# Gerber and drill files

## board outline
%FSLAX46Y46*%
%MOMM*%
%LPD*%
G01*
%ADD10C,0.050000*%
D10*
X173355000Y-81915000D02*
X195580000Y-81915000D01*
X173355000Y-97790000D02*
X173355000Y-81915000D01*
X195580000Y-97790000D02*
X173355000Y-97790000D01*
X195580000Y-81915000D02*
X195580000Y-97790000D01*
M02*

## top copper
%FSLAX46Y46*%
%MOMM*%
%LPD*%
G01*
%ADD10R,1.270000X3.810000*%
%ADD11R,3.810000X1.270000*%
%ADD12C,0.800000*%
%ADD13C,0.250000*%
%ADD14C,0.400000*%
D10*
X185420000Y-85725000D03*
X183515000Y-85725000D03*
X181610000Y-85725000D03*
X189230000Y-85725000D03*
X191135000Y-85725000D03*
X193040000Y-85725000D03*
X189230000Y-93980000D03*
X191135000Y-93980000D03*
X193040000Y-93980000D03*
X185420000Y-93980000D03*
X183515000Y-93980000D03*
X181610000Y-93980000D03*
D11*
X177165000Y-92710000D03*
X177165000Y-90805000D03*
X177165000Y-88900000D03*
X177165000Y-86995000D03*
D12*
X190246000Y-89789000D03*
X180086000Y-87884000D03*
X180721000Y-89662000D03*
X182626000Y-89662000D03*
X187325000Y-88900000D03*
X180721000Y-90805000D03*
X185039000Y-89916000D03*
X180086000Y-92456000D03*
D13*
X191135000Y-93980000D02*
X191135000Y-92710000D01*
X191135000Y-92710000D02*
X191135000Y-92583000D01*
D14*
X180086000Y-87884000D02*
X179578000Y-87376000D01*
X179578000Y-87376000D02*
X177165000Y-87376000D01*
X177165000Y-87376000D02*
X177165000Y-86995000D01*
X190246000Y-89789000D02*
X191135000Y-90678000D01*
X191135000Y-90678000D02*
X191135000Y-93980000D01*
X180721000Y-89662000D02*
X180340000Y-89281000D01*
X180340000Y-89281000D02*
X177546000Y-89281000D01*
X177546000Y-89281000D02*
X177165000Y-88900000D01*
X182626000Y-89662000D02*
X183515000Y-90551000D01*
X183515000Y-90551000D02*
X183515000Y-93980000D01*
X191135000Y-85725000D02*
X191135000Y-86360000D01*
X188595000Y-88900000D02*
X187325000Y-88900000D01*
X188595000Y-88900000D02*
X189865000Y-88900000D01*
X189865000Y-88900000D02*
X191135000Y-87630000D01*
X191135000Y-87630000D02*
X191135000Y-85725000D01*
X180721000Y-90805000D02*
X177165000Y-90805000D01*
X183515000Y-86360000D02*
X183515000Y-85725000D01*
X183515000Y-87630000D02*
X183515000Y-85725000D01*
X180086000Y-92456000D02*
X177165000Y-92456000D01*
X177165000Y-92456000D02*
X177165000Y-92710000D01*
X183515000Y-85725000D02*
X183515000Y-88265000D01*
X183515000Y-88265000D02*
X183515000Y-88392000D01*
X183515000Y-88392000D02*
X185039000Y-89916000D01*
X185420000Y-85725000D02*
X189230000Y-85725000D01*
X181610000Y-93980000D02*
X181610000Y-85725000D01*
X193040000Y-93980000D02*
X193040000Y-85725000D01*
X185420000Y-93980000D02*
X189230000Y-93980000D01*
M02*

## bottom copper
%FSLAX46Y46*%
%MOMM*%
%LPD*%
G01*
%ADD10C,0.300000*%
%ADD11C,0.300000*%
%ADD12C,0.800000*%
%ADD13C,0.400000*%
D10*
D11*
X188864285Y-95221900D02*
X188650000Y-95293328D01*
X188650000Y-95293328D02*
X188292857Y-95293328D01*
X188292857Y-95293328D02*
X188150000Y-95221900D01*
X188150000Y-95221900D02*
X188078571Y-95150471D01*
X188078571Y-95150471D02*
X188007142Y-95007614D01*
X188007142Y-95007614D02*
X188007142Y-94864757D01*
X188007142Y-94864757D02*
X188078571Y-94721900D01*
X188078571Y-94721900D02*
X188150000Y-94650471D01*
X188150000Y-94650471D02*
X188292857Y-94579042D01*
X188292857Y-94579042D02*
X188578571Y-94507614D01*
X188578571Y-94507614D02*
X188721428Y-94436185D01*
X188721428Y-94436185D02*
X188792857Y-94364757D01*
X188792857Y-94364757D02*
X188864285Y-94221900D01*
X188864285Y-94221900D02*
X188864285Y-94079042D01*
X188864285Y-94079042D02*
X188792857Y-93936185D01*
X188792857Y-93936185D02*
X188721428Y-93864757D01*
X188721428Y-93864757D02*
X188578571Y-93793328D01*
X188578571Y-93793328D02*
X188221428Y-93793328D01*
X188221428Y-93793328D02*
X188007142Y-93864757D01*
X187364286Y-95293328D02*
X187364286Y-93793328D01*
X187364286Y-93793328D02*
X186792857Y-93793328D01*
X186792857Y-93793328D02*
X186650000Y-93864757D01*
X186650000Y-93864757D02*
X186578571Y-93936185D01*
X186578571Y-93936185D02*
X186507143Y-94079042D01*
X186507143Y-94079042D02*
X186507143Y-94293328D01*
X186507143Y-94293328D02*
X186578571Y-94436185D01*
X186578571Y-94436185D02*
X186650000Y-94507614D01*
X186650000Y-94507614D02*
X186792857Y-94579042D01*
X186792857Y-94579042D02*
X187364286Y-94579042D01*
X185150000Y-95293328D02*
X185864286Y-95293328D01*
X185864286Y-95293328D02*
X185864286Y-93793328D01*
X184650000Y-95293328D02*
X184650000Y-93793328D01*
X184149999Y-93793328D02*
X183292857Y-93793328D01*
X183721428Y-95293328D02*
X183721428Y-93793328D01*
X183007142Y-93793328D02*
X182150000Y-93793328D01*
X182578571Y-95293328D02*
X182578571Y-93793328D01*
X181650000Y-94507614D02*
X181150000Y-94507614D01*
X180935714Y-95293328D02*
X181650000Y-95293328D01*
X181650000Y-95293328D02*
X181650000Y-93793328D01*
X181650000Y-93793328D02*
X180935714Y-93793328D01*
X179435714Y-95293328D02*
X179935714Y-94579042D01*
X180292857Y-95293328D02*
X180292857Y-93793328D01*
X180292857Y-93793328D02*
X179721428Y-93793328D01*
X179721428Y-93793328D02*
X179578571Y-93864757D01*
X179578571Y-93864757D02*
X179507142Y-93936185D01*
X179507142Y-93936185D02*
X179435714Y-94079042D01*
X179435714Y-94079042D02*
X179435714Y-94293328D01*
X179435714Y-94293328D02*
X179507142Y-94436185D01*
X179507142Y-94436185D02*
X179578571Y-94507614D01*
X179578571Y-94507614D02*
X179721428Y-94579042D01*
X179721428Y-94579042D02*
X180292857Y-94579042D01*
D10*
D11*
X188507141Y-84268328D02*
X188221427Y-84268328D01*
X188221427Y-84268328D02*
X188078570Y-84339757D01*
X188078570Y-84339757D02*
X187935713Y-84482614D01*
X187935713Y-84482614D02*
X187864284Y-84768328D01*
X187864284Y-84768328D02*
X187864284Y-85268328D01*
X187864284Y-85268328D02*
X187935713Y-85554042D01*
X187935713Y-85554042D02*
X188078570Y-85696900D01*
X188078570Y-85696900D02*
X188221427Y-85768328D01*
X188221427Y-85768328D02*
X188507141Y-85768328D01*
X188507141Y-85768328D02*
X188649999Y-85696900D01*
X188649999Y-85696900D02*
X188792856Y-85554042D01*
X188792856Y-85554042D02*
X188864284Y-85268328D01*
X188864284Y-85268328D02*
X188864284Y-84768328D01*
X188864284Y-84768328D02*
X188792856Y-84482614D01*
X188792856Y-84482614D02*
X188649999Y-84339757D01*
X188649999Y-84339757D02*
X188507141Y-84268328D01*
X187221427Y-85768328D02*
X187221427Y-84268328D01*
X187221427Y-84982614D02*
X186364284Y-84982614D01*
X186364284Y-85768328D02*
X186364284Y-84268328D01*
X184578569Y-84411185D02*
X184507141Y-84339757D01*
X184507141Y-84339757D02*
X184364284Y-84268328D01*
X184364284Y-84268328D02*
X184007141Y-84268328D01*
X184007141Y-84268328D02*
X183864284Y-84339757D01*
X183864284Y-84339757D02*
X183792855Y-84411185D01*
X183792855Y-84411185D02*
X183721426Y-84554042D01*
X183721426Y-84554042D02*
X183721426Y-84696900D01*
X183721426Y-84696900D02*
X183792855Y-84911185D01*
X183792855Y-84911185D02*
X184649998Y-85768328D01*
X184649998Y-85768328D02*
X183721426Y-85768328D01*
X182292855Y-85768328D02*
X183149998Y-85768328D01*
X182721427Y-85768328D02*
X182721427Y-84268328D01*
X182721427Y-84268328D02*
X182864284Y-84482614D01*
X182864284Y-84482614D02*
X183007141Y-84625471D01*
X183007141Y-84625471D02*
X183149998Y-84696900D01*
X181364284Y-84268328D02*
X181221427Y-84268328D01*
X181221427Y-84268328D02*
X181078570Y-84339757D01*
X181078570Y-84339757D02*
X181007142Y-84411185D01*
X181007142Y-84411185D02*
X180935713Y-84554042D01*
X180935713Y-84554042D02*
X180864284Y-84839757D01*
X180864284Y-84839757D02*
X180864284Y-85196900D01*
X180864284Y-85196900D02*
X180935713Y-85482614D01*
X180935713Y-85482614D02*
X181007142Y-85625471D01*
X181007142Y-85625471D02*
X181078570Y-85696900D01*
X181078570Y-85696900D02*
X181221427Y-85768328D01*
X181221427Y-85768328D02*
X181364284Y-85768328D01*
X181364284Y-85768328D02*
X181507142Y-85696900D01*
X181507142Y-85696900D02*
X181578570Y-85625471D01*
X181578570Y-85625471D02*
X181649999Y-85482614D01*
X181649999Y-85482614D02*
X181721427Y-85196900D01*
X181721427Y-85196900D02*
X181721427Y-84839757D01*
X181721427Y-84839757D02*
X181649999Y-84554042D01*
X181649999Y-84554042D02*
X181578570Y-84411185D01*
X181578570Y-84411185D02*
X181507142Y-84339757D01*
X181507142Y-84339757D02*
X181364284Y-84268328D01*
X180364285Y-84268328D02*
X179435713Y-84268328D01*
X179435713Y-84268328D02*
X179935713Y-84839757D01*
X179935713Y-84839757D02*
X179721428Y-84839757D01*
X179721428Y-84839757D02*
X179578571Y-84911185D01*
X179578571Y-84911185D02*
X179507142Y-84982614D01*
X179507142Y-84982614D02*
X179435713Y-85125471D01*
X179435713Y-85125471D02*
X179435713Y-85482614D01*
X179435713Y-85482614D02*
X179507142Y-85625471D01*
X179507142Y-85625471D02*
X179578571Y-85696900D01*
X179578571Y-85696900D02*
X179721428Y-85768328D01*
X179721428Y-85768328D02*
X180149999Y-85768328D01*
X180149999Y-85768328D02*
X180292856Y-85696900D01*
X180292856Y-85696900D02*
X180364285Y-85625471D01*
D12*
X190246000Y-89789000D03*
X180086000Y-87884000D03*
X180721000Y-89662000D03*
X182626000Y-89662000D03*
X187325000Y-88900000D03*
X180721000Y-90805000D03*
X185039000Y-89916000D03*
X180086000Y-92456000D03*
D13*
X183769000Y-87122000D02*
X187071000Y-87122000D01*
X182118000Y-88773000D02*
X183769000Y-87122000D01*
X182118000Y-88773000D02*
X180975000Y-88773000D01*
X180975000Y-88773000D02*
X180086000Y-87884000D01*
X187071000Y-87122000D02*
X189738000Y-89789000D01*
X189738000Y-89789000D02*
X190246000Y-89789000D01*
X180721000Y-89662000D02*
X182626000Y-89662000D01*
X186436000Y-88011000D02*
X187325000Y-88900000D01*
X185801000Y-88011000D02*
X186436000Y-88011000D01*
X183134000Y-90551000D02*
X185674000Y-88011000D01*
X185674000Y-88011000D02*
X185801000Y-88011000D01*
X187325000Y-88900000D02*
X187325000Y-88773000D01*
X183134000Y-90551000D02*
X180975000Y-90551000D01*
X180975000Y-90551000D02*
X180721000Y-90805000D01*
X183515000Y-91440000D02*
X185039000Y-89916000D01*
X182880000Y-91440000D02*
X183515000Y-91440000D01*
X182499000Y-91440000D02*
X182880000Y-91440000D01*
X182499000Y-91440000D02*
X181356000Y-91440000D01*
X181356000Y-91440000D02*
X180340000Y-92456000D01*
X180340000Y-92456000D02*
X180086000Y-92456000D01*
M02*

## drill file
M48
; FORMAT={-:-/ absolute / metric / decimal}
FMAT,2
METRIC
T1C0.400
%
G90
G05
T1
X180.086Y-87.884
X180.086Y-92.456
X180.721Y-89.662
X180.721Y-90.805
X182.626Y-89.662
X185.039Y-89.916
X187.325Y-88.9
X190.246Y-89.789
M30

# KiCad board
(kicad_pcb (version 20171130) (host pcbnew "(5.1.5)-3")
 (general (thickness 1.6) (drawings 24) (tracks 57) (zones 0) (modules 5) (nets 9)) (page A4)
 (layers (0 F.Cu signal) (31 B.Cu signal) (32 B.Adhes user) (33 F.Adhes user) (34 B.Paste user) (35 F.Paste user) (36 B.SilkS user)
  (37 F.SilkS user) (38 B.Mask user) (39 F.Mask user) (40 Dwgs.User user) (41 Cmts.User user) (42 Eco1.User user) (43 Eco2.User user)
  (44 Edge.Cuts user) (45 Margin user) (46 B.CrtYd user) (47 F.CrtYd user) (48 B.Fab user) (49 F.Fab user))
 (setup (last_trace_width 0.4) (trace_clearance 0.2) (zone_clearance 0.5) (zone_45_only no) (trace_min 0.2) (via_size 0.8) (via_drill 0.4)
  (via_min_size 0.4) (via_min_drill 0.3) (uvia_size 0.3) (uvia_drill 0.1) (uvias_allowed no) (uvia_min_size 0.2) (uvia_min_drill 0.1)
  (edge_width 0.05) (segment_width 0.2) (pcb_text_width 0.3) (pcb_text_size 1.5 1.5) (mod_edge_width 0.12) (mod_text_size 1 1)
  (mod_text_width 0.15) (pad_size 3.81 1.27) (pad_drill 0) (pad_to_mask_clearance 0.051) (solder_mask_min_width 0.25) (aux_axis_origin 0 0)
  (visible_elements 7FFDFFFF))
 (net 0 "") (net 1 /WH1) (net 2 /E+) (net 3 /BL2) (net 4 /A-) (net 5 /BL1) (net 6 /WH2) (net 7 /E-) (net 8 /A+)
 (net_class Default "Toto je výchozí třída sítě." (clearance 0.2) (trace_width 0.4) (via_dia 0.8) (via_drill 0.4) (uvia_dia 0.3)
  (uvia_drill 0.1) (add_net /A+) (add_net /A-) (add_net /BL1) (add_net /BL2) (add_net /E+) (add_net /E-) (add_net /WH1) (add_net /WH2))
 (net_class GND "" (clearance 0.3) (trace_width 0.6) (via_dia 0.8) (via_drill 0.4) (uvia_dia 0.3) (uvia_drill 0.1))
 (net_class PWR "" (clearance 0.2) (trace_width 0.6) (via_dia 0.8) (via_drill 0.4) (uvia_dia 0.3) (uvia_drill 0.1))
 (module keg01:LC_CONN (layer F.Cu) (at 183.515 85.725 90)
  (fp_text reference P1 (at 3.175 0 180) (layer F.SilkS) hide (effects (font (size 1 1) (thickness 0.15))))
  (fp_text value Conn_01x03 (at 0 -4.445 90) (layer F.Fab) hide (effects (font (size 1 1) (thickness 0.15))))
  (pad 3 smd rect (at 0 1.905 90) (size 3.81 1.27) (layers F.Cu F.Paste F.Mask) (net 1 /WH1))
  (pad 2 smd rect (at 0 0 90) (size 3.81 1.27) (layers F.Cu F.Paste F.Mask) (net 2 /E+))
  (pad 1 smd rect (at 0 -1.905 90) (size 3.81 1.27) (layers F.Cu F.Paste F.Mask) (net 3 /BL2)))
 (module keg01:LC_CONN (layer F.Cu) (at 191.135 85.725 90)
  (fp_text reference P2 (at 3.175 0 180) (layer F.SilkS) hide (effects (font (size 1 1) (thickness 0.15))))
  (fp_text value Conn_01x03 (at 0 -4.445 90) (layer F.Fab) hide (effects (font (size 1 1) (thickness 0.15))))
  (pad 1 smd rect (at 0 -1.905 90) (size 3.81 1.27) (layers F.Cu F.Paste F.Mask) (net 1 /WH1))
  (pad 2 smd rect (at 0 0 90) (size 3.81 1.27) (layers F.Cu F.Paste F.Mask) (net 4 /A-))
  (pad 3 smd rect (at 0 1.905 90) (size 3.81 1.27) (layers F.Cu F.Paste F.Mask) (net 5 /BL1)))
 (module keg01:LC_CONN (layer F.Cu) (at 191.135 93.98 270)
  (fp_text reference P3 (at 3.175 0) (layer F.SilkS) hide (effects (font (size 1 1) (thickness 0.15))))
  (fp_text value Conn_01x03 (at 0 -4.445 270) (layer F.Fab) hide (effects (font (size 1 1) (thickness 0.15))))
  (pad 3 smd rect (at 0 1.905 270) (size 3.81 1.27) (layers F.Cu F.Paste F.Mask) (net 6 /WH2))
  (pad 2 smd rect (at 0 0 270) (size 3.81 1.27) (layers F.Cu F.Paste F.Mask) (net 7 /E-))
  (pad 1 smd rect (at 0 -1.905 270) (size 3.81 1.27) (layers F.Cu F.Paste F.Mask) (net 5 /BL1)))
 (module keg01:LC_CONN (layer F.Cu) (at 183.515 93.98 270)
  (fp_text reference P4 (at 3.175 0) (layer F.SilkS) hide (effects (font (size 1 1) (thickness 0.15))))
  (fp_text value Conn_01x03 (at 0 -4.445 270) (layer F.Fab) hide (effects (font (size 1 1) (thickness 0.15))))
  (pad 1 smd rect (at 0 -1.905 270) (size 3.81 1.27) (layers F.Cu F.Paste F.Mask) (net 6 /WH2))
  (pad 2 smd rect (at 0 0 270) (size 3.81 1.27) (layers F.Cu F.Paste F.Mask) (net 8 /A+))
  (pad 3 smd rect (at 0 1.905 270) (size 3.81 1.27) (layers F.Cu F.Paste F.Mask) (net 3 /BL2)))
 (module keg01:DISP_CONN (layer F.Cu) (at 177.165 90.17 180)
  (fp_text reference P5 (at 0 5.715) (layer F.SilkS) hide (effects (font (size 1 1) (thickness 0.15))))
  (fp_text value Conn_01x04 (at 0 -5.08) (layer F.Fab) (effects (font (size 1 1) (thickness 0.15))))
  (pad 4 smd rect (at 0 -2.54 180) (size 3.81 1.27) (layers F.Cu F.Paste F.Mask) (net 2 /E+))
  (pad 3 smd rect (at 0 -0.635 180) (size 3.81 1.27) (layers F.Cu F.Paste F.Mask) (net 4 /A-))
  (pad 2 smd rect (at 0 1.27 180) (size 3.81 1.27) (layers F.Cu F.Paste F.Mask) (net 8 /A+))
  (pad 1 smd rect (at 0 3.175 180) (size 3.81 1.27) (layers F.Cu F.Paste F.Mask) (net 7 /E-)))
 (gr_line (start 173.355 81.915) (end 195.58 81.915) (angle 90) (layer Edge.Cuts) (width 0.05))
 (gr_line (start 173.355 97.79) (end 173.355 81.915) (angle 90) (layer Edge.Cuts) (width 0.05))
 (gr_line (start 195.58 97.79) (end 173.355 97.79) (angle 90) (layer Edge.Cuts) (width 0.05))
 (gr_line (start 195.58 81.915) (end 195.58 97.79) (angle 90) (layer Edge.Cuts) (width 0.05))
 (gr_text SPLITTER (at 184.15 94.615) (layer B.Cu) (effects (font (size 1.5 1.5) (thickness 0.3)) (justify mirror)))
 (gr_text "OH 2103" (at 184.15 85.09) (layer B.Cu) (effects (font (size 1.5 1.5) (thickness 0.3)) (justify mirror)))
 (segment (start 191.135 93.98) (end 191.135 92.71) (width 0.25) (layer F.Cu) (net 7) (status 400030))
 (segment (start 191.135 92.71) (end 191.135 92.583) (width 0.25) (layer F.Cu) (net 7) (status 30))
 (via (at 190.246 89.789) (size 0.8) (drill 0.4) (layers F.Cu B.Cu) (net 7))
 (segment (start 183.769 87.122) (end 187.071 87.122) (width 0.4) (layer B.Cu) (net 7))
 (segment (start 182.118 88.773) (end 183.769 87.122) (width 0.4) (layer B.Cu) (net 7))
 (segment (start 182.118 88.773) (end 180.975 88.773) (width 0.4) (layer B.Cu) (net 7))
 (segment (start 180.975 88.773) (end 180.086 87.884) (width 0.4) (layer B.Cu) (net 7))
 (via (at 180.086 87.884) (size 0.8) (drill 0.4) (layers F.Cu B.Cu) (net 7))
 (segment (start 180.086 87.884) (end 179.578 87.376) (width 0.4) (layer F.Cu) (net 7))
 (segment (start 179.578 87.376) (end 177.165 87.376) (width 0.4) (layer F.Cu) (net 7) (status 800000))
 (segment (start 177.165 87.376) (end 177.165 86.995) (width 0.4) (layer F.Cu) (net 7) (status C00000))
 (segment (start 190.246 89.789) (end 191.135 90.678) (width 0.4) (layer F.Cu) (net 7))
 (segment (start 191.135 90.678) (end 191.135 93.98) (width 0.4) (layer F.Cu) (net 7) (status 800000))
 (segment (start 187.071 87.122) (end 189.738 89.789) (width 0.4) (layer B.Cu) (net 7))
 (segment (start 189.738 89.789) (end 190.246 89.789) (width 0.4) (layer B.Cu) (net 7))
 (segment (start 180.721 89.662) (end 182.626 89.662) (width 0.4) (layer B.Cu) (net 8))
 (via (at 180.721 89.662) (size 0.8) (drill 0.4) (layers F.Cu B.Cu) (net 8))
 (segment (start 180.721 89.662) (end 180.34 89.281) (width 0.4) (layer F.Cu) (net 8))
 (segment (start 180.34 89.281) (end 177.546 89.281) (width 0.4) (layer F.Cu) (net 8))
 (segment (start 177.546 89.281) (end 177.165 88.9) (width 0.4) (layer F.Cu) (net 8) (status 800000))
 (via (at 182.626 89.662) (size 0.8) (drill 0.4) (layers F.Cu B.Cu) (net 8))
 (segment (start 182.626 89.662) (end 183.515 90.551) (width 0.4) (layer F.Cu) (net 8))
 (segment (start 183.515 90.551) (end 183.515 93.98) (width 0.4) (layer F.Cu) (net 8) (status 800000))
 (segment (start 186.436 88.011) (end 187.325 88.9) (width 0.4) (layer B.Cu) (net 4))
 (segment (start 185.801 88.011) (end 186.436 88.011) (width 0.4) (layer B.Cu) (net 4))
 (segment (start 183.134 90.551) (end 185.674 88.011) (width 0.4) (layer B.Cu) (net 4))
 (segment (start 185.674 88.011) (end 185.801 88.011) (width 0.4) (layer B.Cu) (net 4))
 (segment (start 191.135 85.725) (end 191.135 86.36) (width 0.4) (layer F.Cu) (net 4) (status 400010))
 (segment (start 187.325 88.9) (end 187.325 88.773) (width 0.4) (layer B.Cu) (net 4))
 (via (at 187.325 88.9) (size 0.8) (drill 0.4) (layers F.Cu B.Cu) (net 4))
 (segment (start 188.595 88.9) (end 187.325 88.9) (width 0.4) (layer F.Cu) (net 4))
 (segment (start 188.595 88.9) (end 189.865 88.9) (width 0.4) (layer F.Cu) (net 4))
 (segment (start 189.865 88.9) (end 191.135 87.63) (width 0.4) (layer F.Cu) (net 4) (status 800000))
 (segment (start 191.135 87.63) (end 191.135 85.725) (width 0.4) (layer F.Cu) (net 4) (status C00000))
 (segment (start 183.134 90.551) (end 180.975 90.551) (width 0.4) (layer B.Cu) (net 4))
 (segment (start 180.975 90.551) (end 180.721 90.805) (width 0.4) (layer B.Cu) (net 4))
 (via (at 180.721 90.805) (size 0.8) (drill 0.4) (layers F.Cu B.Cu) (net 4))
 (segment (start 180.721 90.805) (end 177.165 90.805) (width 0.4) (layer F.Cu) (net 4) (status 800000))
 (segment (start 183.515 91.44) (end 185.039 89.916) (width 0.4) (layer B.Cu) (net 2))
 (segment (start 182.88 91.44) (end 183.515 91.44) (width 0.4) (layer B.Cu) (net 2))
 (via (at 185.039 89.916) (size 0.8) (drill 0.4) (layers F.Cu B.Cu) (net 2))
 (segment (start 183.515 86.36) (end 183.515 85.725) (width 0.4) (layer F.Cu) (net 2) (status 800020))
 (segment (start 182.499 91.44) (end 182.88 91.44) (width 0.4) (layer B.Cu) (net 2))
 (segment (start 183.515 87.63) (end 183.515 85.725) (width 0.4) (layer F.Cu) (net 2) (status C00000))
 (segment (start 182.499 91.44) (end 181.356 91.44) (width 0.4) (layer B.Cu) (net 2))
 (via (at 180.086 92.456) (size 0.8) (drill 0.4) (layers F.Cu B.Cu) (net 2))
 (segment (start 180.086 92.456) (end 177.165 92.456) (width 0.4) (layer F.Cu) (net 2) (status 800000))
 (segment (start 177.165 92.456) (end 177.165 92.71) (width 0.4) (layer F.Cu) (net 2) (status C00000))
 (segment (start 183.515 85.725) (end 183.515 88.265) (width 0.4) (layer F.Cu) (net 2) (status 400000))
 (segment (start 183.515 88.265) (end 183.515 88.392) (width 0.4) (layer F.Cu) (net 2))
 (segment (start 183.515 88.392) (end 185.039 89.916) (width 0.4) (layer F.Cu) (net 2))
 (segment (start 181.356 91.44) (end 180.34 92.456) (width 0.4) (layer B.Cu) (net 2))
 (segment (start 180.34 92.456) (end 180.086 92.456) (width 0.4) (layer B.Cu) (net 2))
 (segment (start 185.42 85.725) (end 189.23 85.725) (width 0.4) (layer F.Cu) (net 1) (status C00000))
 (segment (start 181.61 93.98) (end 181.61 85.725) (width 0.4) (layer F.Cu) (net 3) (status C00020))
 (segment (start 193.04 93.98) (end 193.04 85.725) (width 0.4) (layer F.Cu) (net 5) (status C00020))
 (segment (start 185.42 93.98) (end 189.23 93.98) (width 0.4) (layer F.Cu) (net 6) (status C00000)))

